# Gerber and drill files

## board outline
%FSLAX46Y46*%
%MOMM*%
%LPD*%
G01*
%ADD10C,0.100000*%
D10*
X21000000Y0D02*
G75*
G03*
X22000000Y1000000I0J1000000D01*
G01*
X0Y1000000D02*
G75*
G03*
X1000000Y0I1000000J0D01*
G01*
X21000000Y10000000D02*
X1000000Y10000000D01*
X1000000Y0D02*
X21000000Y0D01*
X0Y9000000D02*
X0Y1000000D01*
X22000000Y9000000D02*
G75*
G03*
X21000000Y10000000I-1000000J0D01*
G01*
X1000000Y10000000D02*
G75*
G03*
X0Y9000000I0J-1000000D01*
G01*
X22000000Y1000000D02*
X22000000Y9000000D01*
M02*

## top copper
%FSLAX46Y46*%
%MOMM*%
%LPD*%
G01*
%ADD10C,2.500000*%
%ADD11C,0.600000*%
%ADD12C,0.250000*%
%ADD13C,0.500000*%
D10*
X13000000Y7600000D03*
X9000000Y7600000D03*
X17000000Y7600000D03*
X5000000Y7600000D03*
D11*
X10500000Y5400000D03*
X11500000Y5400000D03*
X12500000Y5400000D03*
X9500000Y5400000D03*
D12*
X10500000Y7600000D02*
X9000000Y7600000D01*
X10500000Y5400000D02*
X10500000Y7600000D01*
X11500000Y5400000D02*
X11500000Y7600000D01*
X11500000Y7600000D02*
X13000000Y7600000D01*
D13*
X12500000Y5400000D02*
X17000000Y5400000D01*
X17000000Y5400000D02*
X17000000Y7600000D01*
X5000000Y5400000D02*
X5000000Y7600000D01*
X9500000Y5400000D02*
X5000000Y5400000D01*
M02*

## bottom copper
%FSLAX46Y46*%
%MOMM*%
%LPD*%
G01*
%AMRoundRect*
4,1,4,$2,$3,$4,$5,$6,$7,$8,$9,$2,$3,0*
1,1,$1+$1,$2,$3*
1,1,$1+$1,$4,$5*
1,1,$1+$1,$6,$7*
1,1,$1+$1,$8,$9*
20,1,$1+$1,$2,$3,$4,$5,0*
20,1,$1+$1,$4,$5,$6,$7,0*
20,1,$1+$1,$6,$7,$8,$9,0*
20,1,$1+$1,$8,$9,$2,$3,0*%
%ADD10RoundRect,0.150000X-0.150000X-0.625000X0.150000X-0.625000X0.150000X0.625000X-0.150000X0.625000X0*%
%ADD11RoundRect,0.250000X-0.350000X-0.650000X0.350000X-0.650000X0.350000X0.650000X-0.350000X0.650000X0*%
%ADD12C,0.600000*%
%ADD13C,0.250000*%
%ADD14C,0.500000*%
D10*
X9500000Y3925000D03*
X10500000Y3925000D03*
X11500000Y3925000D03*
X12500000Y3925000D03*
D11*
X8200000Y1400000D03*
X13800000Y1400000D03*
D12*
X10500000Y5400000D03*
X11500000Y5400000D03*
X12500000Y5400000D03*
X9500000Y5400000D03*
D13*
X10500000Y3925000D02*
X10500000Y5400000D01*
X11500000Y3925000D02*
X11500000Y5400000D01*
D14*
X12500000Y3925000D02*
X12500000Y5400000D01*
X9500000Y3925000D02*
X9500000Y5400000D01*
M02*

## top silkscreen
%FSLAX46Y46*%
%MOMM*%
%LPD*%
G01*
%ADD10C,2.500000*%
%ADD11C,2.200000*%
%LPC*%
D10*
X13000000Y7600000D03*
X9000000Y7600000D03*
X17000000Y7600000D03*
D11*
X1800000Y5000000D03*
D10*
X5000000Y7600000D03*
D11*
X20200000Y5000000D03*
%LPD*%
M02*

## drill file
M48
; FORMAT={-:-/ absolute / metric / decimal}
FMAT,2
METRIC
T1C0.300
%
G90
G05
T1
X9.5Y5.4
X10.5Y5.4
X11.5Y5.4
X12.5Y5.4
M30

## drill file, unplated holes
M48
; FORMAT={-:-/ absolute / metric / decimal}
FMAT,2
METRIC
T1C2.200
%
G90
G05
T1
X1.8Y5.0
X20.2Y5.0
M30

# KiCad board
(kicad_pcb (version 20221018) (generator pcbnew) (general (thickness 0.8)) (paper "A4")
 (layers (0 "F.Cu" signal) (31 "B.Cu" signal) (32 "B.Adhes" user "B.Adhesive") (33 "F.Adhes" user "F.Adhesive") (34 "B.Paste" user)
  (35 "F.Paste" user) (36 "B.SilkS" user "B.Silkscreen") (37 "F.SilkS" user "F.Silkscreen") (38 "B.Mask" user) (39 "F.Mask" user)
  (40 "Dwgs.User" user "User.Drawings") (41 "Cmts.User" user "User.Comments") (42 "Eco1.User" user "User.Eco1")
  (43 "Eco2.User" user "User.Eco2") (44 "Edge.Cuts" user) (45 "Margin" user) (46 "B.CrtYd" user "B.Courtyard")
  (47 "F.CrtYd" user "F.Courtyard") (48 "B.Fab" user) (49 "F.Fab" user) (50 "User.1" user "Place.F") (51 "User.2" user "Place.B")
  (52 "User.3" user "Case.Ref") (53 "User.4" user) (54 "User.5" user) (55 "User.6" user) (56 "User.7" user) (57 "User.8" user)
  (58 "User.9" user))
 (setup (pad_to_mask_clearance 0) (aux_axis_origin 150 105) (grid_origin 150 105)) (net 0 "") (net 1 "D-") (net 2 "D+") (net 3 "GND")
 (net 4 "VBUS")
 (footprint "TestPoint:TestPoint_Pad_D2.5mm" (layer "F.Cu") (at 163 97.4)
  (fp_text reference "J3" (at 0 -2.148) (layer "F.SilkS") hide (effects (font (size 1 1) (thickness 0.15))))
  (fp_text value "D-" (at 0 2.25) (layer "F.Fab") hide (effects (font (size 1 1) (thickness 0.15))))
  (pad "1" smd circle (at 0 0) (size 2.5 2.5) (layers "F.Cu" "F.Mask") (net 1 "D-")))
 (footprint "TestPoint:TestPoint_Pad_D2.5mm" (layer "F.Cu") (at 159 97.4)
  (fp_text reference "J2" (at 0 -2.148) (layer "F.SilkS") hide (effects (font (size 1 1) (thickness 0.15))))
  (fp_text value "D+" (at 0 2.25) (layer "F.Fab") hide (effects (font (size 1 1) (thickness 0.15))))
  (pad "1" smd circle (at 0 0) (size 2.5 2.5) (layers "F.Cu" "F.Mask") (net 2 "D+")))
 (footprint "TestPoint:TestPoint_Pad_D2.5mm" (layer "F.Cu") (at 167 97.4)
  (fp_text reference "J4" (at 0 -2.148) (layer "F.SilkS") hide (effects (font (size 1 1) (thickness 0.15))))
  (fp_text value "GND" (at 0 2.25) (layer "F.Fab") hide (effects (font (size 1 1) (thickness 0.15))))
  (pad "1" smd circle (at 0 0) (size 2.5 2.5) (layers "F.Cu" "F.Mask") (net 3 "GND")))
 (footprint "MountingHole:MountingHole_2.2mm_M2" (layer "F.Cu") (at 151.8 100)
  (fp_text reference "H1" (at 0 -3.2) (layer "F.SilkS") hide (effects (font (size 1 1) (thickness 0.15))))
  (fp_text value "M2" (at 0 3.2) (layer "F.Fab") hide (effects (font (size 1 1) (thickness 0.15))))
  (pad "" np_thru_hole circle (at 0 0) (size 2.2 2.2) (drill 2.2) (layers "*.Cu" "*.Mask")))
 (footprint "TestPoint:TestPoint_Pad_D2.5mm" (layer "F.Cu") (at 155 97.4)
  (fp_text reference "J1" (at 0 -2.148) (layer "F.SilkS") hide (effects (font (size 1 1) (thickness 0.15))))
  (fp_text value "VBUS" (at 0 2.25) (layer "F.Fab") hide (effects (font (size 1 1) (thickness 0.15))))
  (pad "1" smd circle (at 0 0) (size 2.5 2.5) (layers "F.Cu" "F.Mask") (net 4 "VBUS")))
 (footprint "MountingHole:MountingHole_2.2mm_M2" (layer "F.Cu") (at 170.2 100)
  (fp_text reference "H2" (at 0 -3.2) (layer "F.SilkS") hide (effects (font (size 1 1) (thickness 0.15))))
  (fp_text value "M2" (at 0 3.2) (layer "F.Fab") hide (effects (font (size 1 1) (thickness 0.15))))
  (pad "" np_thru_hole circle (at 0 0) (size 2.2 2.2) (drill 2.2) (layers "*.Cu" "*.Mask")))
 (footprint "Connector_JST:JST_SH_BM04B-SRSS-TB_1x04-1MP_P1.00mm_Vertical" (layer "B.Cu") (at 161 102.4)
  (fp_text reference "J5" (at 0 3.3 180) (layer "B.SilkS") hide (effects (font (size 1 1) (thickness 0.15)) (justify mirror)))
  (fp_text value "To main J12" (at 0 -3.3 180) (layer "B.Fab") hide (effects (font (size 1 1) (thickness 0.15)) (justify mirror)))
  (pad "1" smd roundrect (at -1.5 -1.325) (size 0.6 1.55) (layers "B.Cu" "B.Paste" "B.Mask") (roundrect_rratio 0.25) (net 4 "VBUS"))
  (pad "2" smd roundrect (at -0.5 -1.325) (size 0.6 1.55) (layers "B.Cu" "B.Paste" "B.Mask") (roundrect_rratio 0.25) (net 2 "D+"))
  (pad "3" smd roundrect (at 0.5 -1.325) (size 0.6 1.55) (layers "B.Cu" "B.Paste" "B.Mask") (roundrect_rratio 0.25) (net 1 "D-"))
  (pad "4" smd roundrect (at 1.5 -1.325) (size 0.6 1.55) (layers "B.Cu" "B.Paste" "B.Mask") (roundrect_rratio 0.25) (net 3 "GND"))
  (pad "MP" smd roundrect (at -2.8 1.2) (size 1.2 1.8) (layers "B.Cu" "B.Paste" "B.Mask") (roundrect_rratio 0.208333))
  (pad "MP" smd roundrect (at 2.8 1.2) (size 1.2 1.8) (layers "B.Cu" "B.Paste" "B.Mask") (roundrect_rratio 0.208333)))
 (gr_arc (start 172 104) (mid 171.707107 104.707107) (end 171 105) (stroke (width 0.1) (type default)) (layer "Edge.Cuts"))
 (gr_arc (start 151 105) (mid 150.292893 104.707107) (end 150 104) (stroke (width 0.1) (type default)) (layer "Edge.Cuts"))
 (gr_line (start 171 95) (end 151 95) (stroke (width 0.1) (type default)) (layer "Edge.Cuts"))
 (gr_line (start 151 105) (end 171 105) (stroke (width 0.1) (type default)) (layer "Edge.Cuts"))
 (gr_line (start 150 96) (end 150 104) (stroke (width 0.1) (type default)) (layer "Edge.Cuts"))
 (gr_arc (start 171 95) (mid 171.707107 95.292893) (end 172 96) (stroke (width 0.1) (type default)) (layer "Edge.Cuts"))
 (gr_arc (start 150 96) (mid 150.292893 95.292893) (end 151 95) (stroke (width 0.1) (type default)) (layer "Edge.Cuts"))
 (gr_line (start 172 104) (end 172 96) (stroke (width 0.1) (type default)) (layer "Edge.Cuts"))
 (segment (start 160.5 97.4) (end 159 97.4) (width 0.25) (layer "F.Cu") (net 2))
 (segment (start 160.5 99.6) (end 160.5 97.4) (width 0.25) (layer "F.Cu") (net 2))
 (via (at 160.5 99.6) (size 0.6) (drill 0.3) (layers "F.Cu" "B.Cu") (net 2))
 (segment (start 160.5 101.075) (end 160.5 99.6) (width 0.25) (layer "B.Cu") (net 2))
 (segment (start 161.5 99.6) (end 161.5 97.4) (width 0.25) (layer "F.Cu") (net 1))
 (segment (start 161.5 97.4) (end 163 97.4) (width 0.25) (layer "F.Cu") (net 1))
 (via (at 161.5 99.6) (size 0.6) (drill 0.3) (layers "F.Cu" "B.Cu") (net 1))
 (segment (start 161.5 101.075) (end 161.5 99.6) (width 0.25) (layer "B.Cu") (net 1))
 (segment (start 162.5 99.6) (end 167 99.6) (width 0.5) (layer "F.Cu") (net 3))
 (segment (start 167 99.6) (end 167 97.4) (width 0.5) (layer "F.Cu") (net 3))
 (via (at 162.5 99.6) (size 0.6) (drill 0.3) (layers "F.Cu" "B.Cu") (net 3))
 (segment (start 162.5 101.075) (end 162.5 99.6) (width 0.5) (layer "B.Cu") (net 3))
 (segment (start 155 99.6) (end 155 97.4) (width 0.5) (layer "F.Cu") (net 4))
 (segment (start 159.5 99.6) (end 155 99.6) (width 0.5) (layer "F.Cu") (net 4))
 (via (at 159.5 99.6) (size 0.6) (drill 0.3) (layers "F.Cu" "B.Cu") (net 4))
 (segment (start 159.5 101.075) (end 159.5 99.6) (width 0.5) (layer "B.Cu") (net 4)))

